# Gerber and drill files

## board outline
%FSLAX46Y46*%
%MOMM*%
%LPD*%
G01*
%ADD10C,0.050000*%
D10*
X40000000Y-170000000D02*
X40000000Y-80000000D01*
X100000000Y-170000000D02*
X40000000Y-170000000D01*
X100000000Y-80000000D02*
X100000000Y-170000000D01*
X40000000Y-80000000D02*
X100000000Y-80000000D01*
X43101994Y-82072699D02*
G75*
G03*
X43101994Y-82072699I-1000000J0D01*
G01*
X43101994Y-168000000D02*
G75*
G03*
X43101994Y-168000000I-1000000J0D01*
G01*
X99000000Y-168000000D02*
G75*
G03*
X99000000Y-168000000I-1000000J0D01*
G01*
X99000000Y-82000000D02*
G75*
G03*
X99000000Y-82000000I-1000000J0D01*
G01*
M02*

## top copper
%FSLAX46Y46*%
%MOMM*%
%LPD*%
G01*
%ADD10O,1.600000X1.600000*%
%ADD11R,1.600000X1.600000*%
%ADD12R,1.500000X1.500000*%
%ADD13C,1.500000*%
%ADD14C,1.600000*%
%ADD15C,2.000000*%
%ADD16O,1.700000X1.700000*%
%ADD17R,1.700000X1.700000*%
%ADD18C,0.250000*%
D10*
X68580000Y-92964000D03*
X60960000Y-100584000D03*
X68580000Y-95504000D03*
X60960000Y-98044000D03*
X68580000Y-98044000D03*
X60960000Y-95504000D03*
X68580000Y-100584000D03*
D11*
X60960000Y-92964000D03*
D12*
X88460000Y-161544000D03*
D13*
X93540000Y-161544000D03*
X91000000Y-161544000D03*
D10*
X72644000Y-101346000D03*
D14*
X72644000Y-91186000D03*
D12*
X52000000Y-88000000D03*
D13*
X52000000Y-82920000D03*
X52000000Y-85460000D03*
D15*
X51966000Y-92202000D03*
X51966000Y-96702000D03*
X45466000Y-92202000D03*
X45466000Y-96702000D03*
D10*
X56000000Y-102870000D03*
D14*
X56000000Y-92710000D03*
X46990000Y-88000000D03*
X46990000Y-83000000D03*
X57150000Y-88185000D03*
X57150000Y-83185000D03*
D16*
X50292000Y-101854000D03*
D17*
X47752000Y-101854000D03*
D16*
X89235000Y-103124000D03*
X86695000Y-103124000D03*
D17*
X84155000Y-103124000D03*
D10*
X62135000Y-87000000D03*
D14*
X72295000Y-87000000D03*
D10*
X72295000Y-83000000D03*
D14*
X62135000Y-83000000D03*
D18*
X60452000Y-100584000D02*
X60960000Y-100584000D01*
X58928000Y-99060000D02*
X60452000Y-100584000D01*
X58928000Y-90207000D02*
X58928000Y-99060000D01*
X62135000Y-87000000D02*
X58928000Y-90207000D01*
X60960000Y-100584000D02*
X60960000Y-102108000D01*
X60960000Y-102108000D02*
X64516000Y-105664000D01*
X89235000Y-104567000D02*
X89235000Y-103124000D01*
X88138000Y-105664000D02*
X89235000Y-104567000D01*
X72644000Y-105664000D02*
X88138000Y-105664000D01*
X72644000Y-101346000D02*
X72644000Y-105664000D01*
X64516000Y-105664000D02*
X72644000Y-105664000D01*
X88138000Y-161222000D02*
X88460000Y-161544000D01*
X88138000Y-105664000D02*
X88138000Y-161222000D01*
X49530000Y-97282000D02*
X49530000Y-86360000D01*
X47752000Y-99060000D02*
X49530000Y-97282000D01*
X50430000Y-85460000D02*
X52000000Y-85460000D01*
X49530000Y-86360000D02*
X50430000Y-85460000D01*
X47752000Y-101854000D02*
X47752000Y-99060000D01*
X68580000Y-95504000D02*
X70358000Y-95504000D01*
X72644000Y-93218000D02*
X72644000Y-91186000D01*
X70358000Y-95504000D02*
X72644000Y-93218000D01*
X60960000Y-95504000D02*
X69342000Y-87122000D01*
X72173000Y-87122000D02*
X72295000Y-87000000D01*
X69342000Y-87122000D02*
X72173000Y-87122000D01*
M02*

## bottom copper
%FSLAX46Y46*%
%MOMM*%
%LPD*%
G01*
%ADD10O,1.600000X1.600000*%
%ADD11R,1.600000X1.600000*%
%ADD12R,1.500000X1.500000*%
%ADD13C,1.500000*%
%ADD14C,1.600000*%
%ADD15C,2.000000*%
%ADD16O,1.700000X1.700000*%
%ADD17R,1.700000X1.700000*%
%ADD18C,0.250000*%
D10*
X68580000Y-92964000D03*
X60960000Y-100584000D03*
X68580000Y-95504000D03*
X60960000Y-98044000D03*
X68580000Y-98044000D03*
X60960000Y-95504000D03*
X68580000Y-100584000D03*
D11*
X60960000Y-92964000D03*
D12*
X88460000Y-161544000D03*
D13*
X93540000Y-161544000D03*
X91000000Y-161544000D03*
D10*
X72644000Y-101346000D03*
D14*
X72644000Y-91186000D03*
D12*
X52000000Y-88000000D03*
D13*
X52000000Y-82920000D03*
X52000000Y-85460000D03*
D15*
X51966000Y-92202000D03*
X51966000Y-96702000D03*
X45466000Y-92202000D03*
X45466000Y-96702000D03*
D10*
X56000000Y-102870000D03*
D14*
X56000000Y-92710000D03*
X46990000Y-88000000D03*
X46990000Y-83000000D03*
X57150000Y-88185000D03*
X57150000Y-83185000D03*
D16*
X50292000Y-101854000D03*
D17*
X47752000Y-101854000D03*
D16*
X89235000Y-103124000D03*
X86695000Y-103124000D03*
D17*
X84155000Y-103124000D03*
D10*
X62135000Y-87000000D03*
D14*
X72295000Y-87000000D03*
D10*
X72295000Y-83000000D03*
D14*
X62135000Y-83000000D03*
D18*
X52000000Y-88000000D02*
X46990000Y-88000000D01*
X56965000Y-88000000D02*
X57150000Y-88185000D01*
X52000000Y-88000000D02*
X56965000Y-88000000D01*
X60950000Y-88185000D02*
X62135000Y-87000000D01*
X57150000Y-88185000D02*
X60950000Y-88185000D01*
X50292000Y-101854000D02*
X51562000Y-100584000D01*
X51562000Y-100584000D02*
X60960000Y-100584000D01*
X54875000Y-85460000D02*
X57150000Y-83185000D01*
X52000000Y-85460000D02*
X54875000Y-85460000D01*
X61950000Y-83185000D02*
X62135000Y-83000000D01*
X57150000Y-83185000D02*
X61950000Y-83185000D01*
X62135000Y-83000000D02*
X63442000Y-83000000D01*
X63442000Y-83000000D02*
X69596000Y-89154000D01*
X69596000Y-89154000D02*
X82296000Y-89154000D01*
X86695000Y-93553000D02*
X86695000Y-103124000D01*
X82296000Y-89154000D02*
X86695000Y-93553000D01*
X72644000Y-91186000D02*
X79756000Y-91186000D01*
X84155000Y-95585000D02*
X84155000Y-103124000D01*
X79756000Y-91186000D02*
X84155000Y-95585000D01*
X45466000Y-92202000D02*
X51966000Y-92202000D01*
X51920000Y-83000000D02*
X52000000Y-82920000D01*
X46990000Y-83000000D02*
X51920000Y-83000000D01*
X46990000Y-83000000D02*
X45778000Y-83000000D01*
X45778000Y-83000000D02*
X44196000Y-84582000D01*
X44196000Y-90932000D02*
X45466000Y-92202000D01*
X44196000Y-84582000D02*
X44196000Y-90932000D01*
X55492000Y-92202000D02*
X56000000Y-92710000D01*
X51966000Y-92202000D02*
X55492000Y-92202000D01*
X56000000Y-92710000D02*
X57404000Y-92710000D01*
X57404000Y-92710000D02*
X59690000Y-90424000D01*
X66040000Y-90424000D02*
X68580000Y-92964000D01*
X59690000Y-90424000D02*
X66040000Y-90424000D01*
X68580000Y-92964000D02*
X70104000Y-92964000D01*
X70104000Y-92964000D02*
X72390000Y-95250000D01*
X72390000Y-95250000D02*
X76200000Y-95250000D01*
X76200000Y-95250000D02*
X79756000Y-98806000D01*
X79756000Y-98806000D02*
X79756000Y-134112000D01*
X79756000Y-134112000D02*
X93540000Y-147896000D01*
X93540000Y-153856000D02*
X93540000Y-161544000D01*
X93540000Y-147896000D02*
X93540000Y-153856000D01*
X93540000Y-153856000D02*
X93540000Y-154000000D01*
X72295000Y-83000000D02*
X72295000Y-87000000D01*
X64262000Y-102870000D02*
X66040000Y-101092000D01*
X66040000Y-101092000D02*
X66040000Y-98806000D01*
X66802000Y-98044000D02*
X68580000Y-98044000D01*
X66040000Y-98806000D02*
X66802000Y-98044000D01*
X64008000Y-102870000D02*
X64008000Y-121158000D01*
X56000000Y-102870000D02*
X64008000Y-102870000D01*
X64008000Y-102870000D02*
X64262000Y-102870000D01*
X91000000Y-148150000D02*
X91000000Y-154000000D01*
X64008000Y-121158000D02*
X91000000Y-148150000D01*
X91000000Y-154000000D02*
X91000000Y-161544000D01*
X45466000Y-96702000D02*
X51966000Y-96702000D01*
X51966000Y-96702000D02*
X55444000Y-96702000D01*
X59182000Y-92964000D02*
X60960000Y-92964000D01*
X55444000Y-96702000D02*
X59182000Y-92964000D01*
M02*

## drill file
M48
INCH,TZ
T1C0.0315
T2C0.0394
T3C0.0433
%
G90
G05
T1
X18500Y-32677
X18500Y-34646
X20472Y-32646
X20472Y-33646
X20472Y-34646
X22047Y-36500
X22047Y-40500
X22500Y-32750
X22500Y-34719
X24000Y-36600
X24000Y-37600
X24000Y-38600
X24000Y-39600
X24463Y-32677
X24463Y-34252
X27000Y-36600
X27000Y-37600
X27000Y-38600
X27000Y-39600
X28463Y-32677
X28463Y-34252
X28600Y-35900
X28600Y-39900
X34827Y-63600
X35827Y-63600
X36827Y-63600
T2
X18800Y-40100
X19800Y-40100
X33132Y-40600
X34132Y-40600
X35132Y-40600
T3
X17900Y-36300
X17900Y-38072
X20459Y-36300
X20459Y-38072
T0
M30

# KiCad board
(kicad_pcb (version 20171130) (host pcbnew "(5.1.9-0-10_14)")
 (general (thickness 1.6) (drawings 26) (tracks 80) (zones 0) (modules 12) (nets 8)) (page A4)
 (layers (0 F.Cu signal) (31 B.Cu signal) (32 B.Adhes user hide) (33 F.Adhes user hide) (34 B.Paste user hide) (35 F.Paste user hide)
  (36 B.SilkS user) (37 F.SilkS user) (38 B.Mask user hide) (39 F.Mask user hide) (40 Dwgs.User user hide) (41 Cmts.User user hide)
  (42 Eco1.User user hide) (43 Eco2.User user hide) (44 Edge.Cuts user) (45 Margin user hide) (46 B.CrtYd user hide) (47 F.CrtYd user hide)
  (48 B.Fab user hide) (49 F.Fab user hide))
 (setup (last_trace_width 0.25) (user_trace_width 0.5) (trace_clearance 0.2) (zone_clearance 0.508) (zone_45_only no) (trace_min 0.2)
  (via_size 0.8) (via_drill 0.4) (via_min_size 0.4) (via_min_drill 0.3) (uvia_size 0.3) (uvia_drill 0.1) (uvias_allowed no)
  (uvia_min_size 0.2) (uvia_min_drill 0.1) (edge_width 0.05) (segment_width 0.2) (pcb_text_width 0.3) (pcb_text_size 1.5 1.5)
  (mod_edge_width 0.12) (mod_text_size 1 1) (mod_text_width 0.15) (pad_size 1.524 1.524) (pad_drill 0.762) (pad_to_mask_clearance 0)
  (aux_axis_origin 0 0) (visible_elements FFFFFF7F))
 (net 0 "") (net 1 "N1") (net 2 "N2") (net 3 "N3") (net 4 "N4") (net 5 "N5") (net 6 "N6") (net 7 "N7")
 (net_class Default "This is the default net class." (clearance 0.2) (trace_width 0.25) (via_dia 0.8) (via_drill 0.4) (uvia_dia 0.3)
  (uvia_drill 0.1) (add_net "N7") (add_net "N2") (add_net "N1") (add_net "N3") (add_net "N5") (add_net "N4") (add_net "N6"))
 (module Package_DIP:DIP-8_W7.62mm (layer F.Cu) (at 60.96 92.964)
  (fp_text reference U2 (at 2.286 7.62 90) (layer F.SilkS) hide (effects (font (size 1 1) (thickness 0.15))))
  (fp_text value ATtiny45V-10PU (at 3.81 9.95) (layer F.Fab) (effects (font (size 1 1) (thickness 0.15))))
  (pad 8 thru_hole oval (at 7.62 0) (size 1.6 1.6) (drill 0.8) (layers *.Cu *.Mask) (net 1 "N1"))
  (pad 4 thru_hole oval (at 0 7.62) (size 1.6 1.6) (drill 0.8) (layers *.Cu *.Mask) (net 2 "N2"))
  (pad 7 thru_hole oval (at 7.62 2.54) (size 1.6 1.6) (drill 0.8) (layers *.Cu *.Mask) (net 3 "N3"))
  (pad 3 thru_hole oval (at 0 5.08) (size 1.6 1.6) (drill 0.8) (layers *.Cu *.Mask))
  (pad 6 thru_hole oval (at 7.62 5.08) (size 1.6 1.6) (drill 0.8) (layers *.Cu *.Mask) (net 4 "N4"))
  (pad 2 thru_hole oval (at 0 2.54) (size 1.6 1.6) (drill 0.8) (layers *.Cu *.Mask) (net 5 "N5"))
  (pad 5 thru_hole oval (at 7.62 7.62) (size 1.6 1.6) (drill 0.8) (layers *.Cu *.Mask))
  (pad 1 thru_hole rect (at 0 0) (size 1.6 1.6) (drill 0.8) (layers *.Cu *.Mask) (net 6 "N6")))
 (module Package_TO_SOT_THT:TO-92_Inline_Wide (layer F.Cu) (at 88.46 161.544)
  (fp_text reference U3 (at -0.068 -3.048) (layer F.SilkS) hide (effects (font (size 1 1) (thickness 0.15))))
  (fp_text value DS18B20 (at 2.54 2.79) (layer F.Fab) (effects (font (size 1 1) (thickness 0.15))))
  (pad 1 thru_hole rect (at 0 0) (size 1.5 1.5) (drill 0.8) (layers *.Cu *.Mask) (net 2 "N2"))
  (pad 3 thru_hole circle (at 5.08 0) (size 1.5 1.5) (drill 0.8) (layers *.Cu *.Mask) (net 1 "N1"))
  (pad 2 thru_hole circle (at 2.54 0) (size 1.5 1.5) (drill 0.8) (layers *.Cu *.Mask) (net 4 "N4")))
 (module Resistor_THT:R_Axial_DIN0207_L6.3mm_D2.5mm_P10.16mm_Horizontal (layer F.Cu) (at 72.644 91.186 270)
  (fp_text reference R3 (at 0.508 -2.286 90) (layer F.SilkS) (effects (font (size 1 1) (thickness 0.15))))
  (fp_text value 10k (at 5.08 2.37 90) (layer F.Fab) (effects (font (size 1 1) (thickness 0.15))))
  (pad 2 thru_hole oval (at 10.16 0 270) (size 1.6 1.6) (drill 0.8) (layers *.Cu *.Mask) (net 2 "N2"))
  (pad 1 thru_hole circle (at 0 0 270) (size 1.6 1.6) (drill 0.8) (layers *.Cu *.Mask) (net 3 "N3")))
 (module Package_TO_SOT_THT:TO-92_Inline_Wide (layer F.Cu) (at 52 88 90)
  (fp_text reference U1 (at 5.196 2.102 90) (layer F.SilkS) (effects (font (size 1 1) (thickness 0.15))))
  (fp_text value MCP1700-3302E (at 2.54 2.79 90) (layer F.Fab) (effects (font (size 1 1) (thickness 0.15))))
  (pad 1 thru_hole rect (at 0 0 90) (size 1.5 1.5) (drill 0.8) (layers *.Cu *.Mask) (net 2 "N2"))
  (pad 3 thru_hole circle (at 5.08 0 90) (size 1.5 1.5) (drill 0.8) (layers *.Cu *.Mask) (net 1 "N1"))
  (pad 2 thru_hole circle (at 2.54 0 90) (size 1.5 1.5) (drill 0.8) (layers *.Cu *.Mask) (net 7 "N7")))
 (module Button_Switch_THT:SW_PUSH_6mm (layer F.Cu) (at 45.466 92.202)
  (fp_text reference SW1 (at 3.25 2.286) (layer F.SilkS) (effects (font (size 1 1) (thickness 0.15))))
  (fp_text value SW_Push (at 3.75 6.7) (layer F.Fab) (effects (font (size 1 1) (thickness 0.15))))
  (pad 1 thru_hole circle (at 6.5 0 90) (size 2 2) (drill 1.1) (layers *.Cu *.Mask) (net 1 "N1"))
  (pad 2 thru_hole circle (at 6.5 4.5 90) (size 2 2) (drill 1.1) (layers *.Cu *.Mask) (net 6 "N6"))
  (pad 1 thru_hole circle (at 0 0 90) (size 2 2) (drill 1.1) (layers *.Cu *.Mask) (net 1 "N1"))
  (pad 2 thru_hole circle (at 0 4.5 90) (size 2 2) (drill 1.1) (layers *.Cu *.Mask) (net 6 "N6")))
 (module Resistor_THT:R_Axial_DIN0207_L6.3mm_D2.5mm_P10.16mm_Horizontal (layer F.Cu) (at 56 92.71 270)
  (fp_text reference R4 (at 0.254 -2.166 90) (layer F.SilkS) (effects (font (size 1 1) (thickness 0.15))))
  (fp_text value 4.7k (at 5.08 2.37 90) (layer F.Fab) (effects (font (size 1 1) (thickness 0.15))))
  (pad 2 thru_hole oval (at 10.16 0 270) (size 1.6 1.6) (drill 0.8) (layers *.Cu *.Mask) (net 4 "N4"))
  (pad 1 thru_hole circle (at 0 0 270) (size 1.6 1.6) (drill 0.8) (layers *.Cu *.Mask) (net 1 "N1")))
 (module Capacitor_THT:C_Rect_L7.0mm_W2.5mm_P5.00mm (layer F.Cu) (at 46.99 83 270)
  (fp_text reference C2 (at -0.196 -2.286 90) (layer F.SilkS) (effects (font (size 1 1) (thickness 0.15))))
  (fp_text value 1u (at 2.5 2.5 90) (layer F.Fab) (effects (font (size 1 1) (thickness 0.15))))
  (pad 2 thru_hole circle (at 5 0 270) (size 1.6 1.6) (drill 0.8) (layers *.Cu *.Mask) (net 2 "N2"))
  (pad 1 thru_hole circle (at 0 0 270) (size 1.6 1.6) (drill 0.8) (layers *.Cu *.Mask) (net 1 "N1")))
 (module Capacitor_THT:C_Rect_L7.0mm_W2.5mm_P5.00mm (layer F.Cu) (at 57.15 83.185 270)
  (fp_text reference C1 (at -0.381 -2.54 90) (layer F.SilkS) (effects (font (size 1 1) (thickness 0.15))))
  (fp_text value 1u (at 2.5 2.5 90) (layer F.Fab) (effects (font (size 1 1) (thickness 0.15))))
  (pad 2 thru_hole circle (at 5 0 270) (size 1.6 1.6) (drill 0.8) (layers *.Cu *.Mask) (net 2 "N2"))
  (pad 1 thru_hole circle (at 0 0 270) (size 1.6 1.6) (drill 0.8) (layers *.Cu *.Mask) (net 7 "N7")))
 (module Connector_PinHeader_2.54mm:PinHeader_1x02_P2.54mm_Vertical (layer F.Cu) (at 47.752 101.854 90)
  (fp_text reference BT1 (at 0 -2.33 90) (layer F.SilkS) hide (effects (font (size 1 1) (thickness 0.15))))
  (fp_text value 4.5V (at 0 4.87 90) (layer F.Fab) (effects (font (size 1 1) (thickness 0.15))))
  (pad 2 thru_hole oval (at 0 2.54 90) (size 1.7 1.7) (drill 1) (layers *.Cu *.Mask) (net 2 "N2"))
  (pad 1 thru_hole rect (at 0 0 90) (size 1.7 1.7) (drill 1) (layers *.Cu *.Mask) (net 7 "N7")))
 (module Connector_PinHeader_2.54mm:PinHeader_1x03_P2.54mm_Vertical (layer F.Cu) (at 84.155 103.124 90)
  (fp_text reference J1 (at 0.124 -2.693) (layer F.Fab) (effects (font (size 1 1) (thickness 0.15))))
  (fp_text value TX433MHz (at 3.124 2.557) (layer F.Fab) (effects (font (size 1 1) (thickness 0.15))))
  (pad 3 thru_hole oval (at 0 5.08 90) (size 1.7 1.7) (drill 1) (layers *.Cu *.Mask) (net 2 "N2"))
  (pad 2 thru_hole oval (at 0 2.54 90) (size 1.7 1.7) (drill 1) (layers *.Cu *.Mask) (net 7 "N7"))
  (pad 1 thru_hole rect (at 0 0 90) (size 1.7 1.7) (drill 1) (layers *.Cu *.Mask) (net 3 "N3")))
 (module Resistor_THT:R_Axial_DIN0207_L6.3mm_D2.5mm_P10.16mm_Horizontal (layer F.Cu) (at 72.295 87 180)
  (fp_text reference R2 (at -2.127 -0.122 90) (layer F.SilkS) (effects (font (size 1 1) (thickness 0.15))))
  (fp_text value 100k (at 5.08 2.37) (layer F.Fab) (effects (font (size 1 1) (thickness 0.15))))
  (pad 2 thru_hole oval (at 10.16 0 180) (size 1.6 1.6) (drill 0.8) (layers *.Cu *.Mask) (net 2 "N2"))
  (pad 1 thru_hole circle (at 0 0 180) (size 1.6 1.6) (drill 0.8) (layers *.Cu *.Mask) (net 5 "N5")))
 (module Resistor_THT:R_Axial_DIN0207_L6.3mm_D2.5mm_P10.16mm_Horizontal (layer F.Cu) (at 62.135 83)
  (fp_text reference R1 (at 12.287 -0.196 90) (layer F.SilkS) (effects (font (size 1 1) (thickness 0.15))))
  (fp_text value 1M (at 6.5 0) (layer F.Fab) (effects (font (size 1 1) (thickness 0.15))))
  (pad 2 thru_hole oval (at 10.16 0) (size 1.6 1.6) (drill 0.8) (layers *.Cu *.Mask) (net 5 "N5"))
  (pad 1 thru_hole circle (at 0 0) (size 1.6 1.6) (drill 0.8) (layers *.Cu *.Mask) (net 7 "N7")))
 (gr_line (start 40 170) (end 40 80) (layer Edge.Cuts) (width 0.05))
 (gr_line (start 100 170) (end 40 170) (layer Edge.Cuts) (width 0.05))
 (gr_line (start 100 80) (end 100 170) (layer Edge.Cuts) (width 0.05))
 (gr_line (start 40 80) (end 100 80) (layer Edge.Cuts) (width 0.05))
 (gr_circle (center 42.101994 82.072699) (end 42.101994 83.072699) (layer Edge.Cuts) (width 0.05))
 (gr_circle (center 42.101994 168) (end 42.101994 169) (layer Edge.Cuts) (width 0.05))
 (gr_circle (center 98 168) (end 98 169) (layer Edge.Cuts) (width 0.05))
 (gr_circle (center 98 82) (end 98 83) (layer Edge.Cuts) (width 0.05))
 (segment (start 52 88) (end 46.99 88) (width 0.25) (layer B.Cu) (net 2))
 (segment (start 56.965 88) (end 57.15 88.185) (width 0.25) (layer B.Cu) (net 2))
 (segment (start 52 88) (end 56.965 88) (width 0.25) (layer B.Cu) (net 2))
 (segment (start 60.95 88.185) (end 62.135 87) (width 0.25) (layer B.Cu) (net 2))
 (segment (start 57.15 88.185) (end 60.95 88.185) (width 0.25) (layer B.Cu) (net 2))
 (segment (start 50.292 101.854) (end 51.562 100.584) (width 0.25) (layer B.Cu) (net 2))
 (segment (start 51.562 100.584) (end 60.96 100.584) (width 0.25) (layer B.Cu) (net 2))
 (segment (start 60.452 100.584) (end 60.96 100.584) (width 0.25) (layer F.Cu) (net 2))
 (segment (start 58.928 99.06) (end 60.452 100.584) (width 0.25) (layer F.Cu) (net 2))
 (segment (start 58.928 90.207) (end 58.928 99.06) (width 0.25) (layer F.Cu) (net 2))
 (segment (start 62.135 87) (end 58.928 90.207) (width 0.25) (layer F.Cu) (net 2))
 (segment (start 60.96 100.584) (end 60.96 102.108) (width 0.25) (layer F.Cu) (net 2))
 (segment (start 60.96 102.108) (end 64.516 105.664) (width 0.25) (layer F.Cu) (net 2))
 (segment (start 89.235 104.567) (end 89.235 103.124) (width 0.25) (layer F.Cu) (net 2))
 (segment (start 88.138 105.664) (end 89.235 104.567) (width 0.25) (layer F.Cu) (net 2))
 (segment (start 72.644 105.664) (end 88.138 105.664) (width 0.25) (layer F.Cu) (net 2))
 (segment (start 72.644 101.346) (end 72.644 105.664) (width 0.25) (layer F.Cu) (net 2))
 (segment (start 64.516 105.664) (end 72.644 105.664) (width 0.25) (layer F.Cu) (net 2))
 (segment (start 88.138 161.222) (end 88.46 161.544) (width 0.25) (layer F.Cu) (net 2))
 (segment (start 88.138 105.664) (end 88.138 161.222) (width 0.25) (layer F.Cu) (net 2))
 (segment (start 49.53 97.282) (end 49.53 86.36) (width 0.25) (layer F.Cu) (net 7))
 (segment (start 47.752 99.06) (end 49.53 97.282) (width 0.25) (layer F.Cu) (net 7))
 (segment (start 50.43 85.46) (end 52 85.46) (width 0.25) (layer F.Cu) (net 7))
 (segment (start 49.53 86.36) (end 50.43 85.46) (width 0.25) (layer F.Cu) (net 7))
 (segment (start 47.752 101.854) (end 47.752 99.06) (width 0.25) (layer F.Cu) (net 7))
 (segment (start 54.875 85.46) (end 57.15 83.185) (width 0.25) (layer B.Cu) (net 7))
 (segment (start 52 85.46) (end 54.875 85.46) (width 0.25) (layer B.Cu) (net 7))
 (segment (start 61.95 83.185) (end 62.135 83) (width 0.25) (layer B.Cu) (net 7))
 (segment (start 57.15 83.185) (end 61.95 83.185) (width 0.25) (layer B.Cu) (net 7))
 (segment (start 62.135 83) (end 63.442 83) (width 0.25) (layer B.Cu) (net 7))
 (segment (start 63.442 83) (end 69.596 89.154) (width 0.25) (layer B.Cu) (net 7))
 (segment (start 69.596 89.154) (end 82.296 89.154) (width 0.25) (layer B.Cu) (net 7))
 (segment (start 86.695 93.553) (end 86.695 103.124) (width 0.25) (layer B.Cu) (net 7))
 (segment (start 82.296 89.154) (end 86.695 93.553) (width 0.25) (layer B.Cu) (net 7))
 (segment (start 72.644 91.186) (end 79.756 91.186) (width 0.25) (layer B.Cu) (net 3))
 (segment (start 84.155 95.585) (end 84.155 103.124) (width 0.25) (layer B.Cu) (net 3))
 (segment (start 79.756 91.186) (end 84.155 95.585) (width 0.25) (layer B.Cu) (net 3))
 (segment (start 68.58 95.504) (end 70.358 95.504) (width 0.25) (layer F.Cu) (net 3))
 (segment (start 72.644 93.218) (end 72.644 91.186) (width 0.25) (layer F.Cu) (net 3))
 (segment (start 70.358 95.504) (end 72.644 93.218) (width 0.25) (layer F.Cu) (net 3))
 (segment (start 45.466 92.202) (end 51.966 92.202) (width 0.25) (layer B.Cu) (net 1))
 (segment (start 51.92 83) (end 52 82.92) (width 0.25) (layer B.Cu) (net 1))
 (segment (start 46.99 83) (end 51.92 83) (width 0.25) (layer B.Cu) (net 1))
 (segment (start 46.99 83) (end 45.778 83) (width 0.25) (layer B.Cu) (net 1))
 (segment (start 45.778 83) (end 44.196 84.582) (width 0.25) (layer B.Cu) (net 1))
 (segment (start 44.196 90.932) (end 45.466 92.202) (width 0.25) (layer B.Cu) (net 1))
 (segment (start 44.196 84.582) (end 44.196 90.932) (width 0.25) (layer B.Cu) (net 1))
 (segment (start 55.492 92.202) (end 56 92.71) (width 0.25) (layer B.Cu) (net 1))
 (segment (start 51.966 92.202) (end 55.492 92.202) (width 0.25) (layer B.Cu) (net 1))
 (segment (start 56 92.71) (end 57.404 92.71) (width 0.25) (layer B.Cu) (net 1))
 (segment (start 57.404 92.71) (end 59.69 90.424) (width 0.25) (layer B.Cu) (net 1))
 (segment (start 66.04 90.424) (end 68.58 92.964) (width 0.25) (layer B.Cu) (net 1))
 (segment (start 59.69 90.424) (end 66.04 90.424) (width 0.25) (layer B.Cu) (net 1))
 (segment (start 68.58 92.964) (end 70.104 92.964) (width 0.25) (layer B.Cu) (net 1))
 (segment (start 70.104 92.964) (end 72.39 95.25) (width 0.25) (layer B.Cu) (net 1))
 (segment (start 72.39 95.25) (end 76.2 95.25) (width 0.25) (layer B.Cu) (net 1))
 (segment (start 76.2 95.25) (end 79.756 98.806) (width 0.25) (layer B.Cu) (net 1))
 (segment (start 79.756 98.806) (end 79.756 134.112) (width 0.25) (layer B.Cu) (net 1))
 (segment (start 79.756 134.112) (end 93.54 147.896) (width 0.25) (layer B.Cu) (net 1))
 (segment (start 93.54 153.856) (end 93.54 161.544) (width 0.25) (layer B.Cu) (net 1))
 (segment (start 93.54 147.896) (end 93.54 153.856) (width 0.25) (layer B.Cu) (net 1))
 (segment (start 93.54 153.856) (end 93.54 154) (width 0.25) (layer B.Cu) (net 1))
 (segment (start 60.96 95.504) (end 69.342 87.122) (width 0.25) (layer F.Cu) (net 5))
 (segment (start 72.173 87.122) (end 72.295 87) (width 0.25) (layer F.Cu) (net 5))
 (segment (start 69.342 87.122) (end 72.173 87.122) (width 0.25) (layer F.Cu) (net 5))
 (segment (start 72.295 83) (end 72.295 87) (width 0.25) (layer B.Cu) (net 5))
 (segment (start 64.262 102.87) (end 66.04 101.092) (width 0.25) (layer B.Cu) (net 4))
 (segment (start 66.04 101.092) (end 66.04 98.806) (width 0.25) (layer B.Cu) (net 4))
 (segment (start 66.802 98.044) (end 68.58 98.044) (width 0.25) (layer B.Cu) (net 4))
 (segment (start 66.04 98.806) (end 66.802 98.044) (width 0.25) (layer B.Cu) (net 4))
 (segment (start 64.008 102.87) (end 64.008 121.158) (width 0.25) (layer B.Cu) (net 4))
 (segment (start 56 102.87) (end 64.008 102.87) (width 0.25) (layer B.Cu) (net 4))
 (segment (start 64.008 102.87) (end 64.262 102.87) (width 0.25) (layer B.Cu) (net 4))
 (segment (start 91 148.15) (end 91 154) (width 0.25) (layer B.Cu) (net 4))
 (segment (start 64.008 121.158) (end 91 148.15) (width 0.25) (layer B.Cu) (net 4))
 (segment (start 91 154) (end 91 161.544) (width 0.25) (layer B.Cu) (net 4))
 (segment (start 45.466 96.702) (end 51.966 96.702) (width 0.25) (layer B.Cu) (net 6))
 (segment (start 51.966 96.702) (end 55.444 96.702) (width 0.25) (layer B.Cu) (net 6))
 (segment (start 59.182 92.964) (end 60.96 92.964) (width 0.25) (layer B.Cu) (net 6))
 (segment (start 55.444 96.702) (end 59.182 92.964) (width 0.25) (layer B.Cu) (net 6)))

